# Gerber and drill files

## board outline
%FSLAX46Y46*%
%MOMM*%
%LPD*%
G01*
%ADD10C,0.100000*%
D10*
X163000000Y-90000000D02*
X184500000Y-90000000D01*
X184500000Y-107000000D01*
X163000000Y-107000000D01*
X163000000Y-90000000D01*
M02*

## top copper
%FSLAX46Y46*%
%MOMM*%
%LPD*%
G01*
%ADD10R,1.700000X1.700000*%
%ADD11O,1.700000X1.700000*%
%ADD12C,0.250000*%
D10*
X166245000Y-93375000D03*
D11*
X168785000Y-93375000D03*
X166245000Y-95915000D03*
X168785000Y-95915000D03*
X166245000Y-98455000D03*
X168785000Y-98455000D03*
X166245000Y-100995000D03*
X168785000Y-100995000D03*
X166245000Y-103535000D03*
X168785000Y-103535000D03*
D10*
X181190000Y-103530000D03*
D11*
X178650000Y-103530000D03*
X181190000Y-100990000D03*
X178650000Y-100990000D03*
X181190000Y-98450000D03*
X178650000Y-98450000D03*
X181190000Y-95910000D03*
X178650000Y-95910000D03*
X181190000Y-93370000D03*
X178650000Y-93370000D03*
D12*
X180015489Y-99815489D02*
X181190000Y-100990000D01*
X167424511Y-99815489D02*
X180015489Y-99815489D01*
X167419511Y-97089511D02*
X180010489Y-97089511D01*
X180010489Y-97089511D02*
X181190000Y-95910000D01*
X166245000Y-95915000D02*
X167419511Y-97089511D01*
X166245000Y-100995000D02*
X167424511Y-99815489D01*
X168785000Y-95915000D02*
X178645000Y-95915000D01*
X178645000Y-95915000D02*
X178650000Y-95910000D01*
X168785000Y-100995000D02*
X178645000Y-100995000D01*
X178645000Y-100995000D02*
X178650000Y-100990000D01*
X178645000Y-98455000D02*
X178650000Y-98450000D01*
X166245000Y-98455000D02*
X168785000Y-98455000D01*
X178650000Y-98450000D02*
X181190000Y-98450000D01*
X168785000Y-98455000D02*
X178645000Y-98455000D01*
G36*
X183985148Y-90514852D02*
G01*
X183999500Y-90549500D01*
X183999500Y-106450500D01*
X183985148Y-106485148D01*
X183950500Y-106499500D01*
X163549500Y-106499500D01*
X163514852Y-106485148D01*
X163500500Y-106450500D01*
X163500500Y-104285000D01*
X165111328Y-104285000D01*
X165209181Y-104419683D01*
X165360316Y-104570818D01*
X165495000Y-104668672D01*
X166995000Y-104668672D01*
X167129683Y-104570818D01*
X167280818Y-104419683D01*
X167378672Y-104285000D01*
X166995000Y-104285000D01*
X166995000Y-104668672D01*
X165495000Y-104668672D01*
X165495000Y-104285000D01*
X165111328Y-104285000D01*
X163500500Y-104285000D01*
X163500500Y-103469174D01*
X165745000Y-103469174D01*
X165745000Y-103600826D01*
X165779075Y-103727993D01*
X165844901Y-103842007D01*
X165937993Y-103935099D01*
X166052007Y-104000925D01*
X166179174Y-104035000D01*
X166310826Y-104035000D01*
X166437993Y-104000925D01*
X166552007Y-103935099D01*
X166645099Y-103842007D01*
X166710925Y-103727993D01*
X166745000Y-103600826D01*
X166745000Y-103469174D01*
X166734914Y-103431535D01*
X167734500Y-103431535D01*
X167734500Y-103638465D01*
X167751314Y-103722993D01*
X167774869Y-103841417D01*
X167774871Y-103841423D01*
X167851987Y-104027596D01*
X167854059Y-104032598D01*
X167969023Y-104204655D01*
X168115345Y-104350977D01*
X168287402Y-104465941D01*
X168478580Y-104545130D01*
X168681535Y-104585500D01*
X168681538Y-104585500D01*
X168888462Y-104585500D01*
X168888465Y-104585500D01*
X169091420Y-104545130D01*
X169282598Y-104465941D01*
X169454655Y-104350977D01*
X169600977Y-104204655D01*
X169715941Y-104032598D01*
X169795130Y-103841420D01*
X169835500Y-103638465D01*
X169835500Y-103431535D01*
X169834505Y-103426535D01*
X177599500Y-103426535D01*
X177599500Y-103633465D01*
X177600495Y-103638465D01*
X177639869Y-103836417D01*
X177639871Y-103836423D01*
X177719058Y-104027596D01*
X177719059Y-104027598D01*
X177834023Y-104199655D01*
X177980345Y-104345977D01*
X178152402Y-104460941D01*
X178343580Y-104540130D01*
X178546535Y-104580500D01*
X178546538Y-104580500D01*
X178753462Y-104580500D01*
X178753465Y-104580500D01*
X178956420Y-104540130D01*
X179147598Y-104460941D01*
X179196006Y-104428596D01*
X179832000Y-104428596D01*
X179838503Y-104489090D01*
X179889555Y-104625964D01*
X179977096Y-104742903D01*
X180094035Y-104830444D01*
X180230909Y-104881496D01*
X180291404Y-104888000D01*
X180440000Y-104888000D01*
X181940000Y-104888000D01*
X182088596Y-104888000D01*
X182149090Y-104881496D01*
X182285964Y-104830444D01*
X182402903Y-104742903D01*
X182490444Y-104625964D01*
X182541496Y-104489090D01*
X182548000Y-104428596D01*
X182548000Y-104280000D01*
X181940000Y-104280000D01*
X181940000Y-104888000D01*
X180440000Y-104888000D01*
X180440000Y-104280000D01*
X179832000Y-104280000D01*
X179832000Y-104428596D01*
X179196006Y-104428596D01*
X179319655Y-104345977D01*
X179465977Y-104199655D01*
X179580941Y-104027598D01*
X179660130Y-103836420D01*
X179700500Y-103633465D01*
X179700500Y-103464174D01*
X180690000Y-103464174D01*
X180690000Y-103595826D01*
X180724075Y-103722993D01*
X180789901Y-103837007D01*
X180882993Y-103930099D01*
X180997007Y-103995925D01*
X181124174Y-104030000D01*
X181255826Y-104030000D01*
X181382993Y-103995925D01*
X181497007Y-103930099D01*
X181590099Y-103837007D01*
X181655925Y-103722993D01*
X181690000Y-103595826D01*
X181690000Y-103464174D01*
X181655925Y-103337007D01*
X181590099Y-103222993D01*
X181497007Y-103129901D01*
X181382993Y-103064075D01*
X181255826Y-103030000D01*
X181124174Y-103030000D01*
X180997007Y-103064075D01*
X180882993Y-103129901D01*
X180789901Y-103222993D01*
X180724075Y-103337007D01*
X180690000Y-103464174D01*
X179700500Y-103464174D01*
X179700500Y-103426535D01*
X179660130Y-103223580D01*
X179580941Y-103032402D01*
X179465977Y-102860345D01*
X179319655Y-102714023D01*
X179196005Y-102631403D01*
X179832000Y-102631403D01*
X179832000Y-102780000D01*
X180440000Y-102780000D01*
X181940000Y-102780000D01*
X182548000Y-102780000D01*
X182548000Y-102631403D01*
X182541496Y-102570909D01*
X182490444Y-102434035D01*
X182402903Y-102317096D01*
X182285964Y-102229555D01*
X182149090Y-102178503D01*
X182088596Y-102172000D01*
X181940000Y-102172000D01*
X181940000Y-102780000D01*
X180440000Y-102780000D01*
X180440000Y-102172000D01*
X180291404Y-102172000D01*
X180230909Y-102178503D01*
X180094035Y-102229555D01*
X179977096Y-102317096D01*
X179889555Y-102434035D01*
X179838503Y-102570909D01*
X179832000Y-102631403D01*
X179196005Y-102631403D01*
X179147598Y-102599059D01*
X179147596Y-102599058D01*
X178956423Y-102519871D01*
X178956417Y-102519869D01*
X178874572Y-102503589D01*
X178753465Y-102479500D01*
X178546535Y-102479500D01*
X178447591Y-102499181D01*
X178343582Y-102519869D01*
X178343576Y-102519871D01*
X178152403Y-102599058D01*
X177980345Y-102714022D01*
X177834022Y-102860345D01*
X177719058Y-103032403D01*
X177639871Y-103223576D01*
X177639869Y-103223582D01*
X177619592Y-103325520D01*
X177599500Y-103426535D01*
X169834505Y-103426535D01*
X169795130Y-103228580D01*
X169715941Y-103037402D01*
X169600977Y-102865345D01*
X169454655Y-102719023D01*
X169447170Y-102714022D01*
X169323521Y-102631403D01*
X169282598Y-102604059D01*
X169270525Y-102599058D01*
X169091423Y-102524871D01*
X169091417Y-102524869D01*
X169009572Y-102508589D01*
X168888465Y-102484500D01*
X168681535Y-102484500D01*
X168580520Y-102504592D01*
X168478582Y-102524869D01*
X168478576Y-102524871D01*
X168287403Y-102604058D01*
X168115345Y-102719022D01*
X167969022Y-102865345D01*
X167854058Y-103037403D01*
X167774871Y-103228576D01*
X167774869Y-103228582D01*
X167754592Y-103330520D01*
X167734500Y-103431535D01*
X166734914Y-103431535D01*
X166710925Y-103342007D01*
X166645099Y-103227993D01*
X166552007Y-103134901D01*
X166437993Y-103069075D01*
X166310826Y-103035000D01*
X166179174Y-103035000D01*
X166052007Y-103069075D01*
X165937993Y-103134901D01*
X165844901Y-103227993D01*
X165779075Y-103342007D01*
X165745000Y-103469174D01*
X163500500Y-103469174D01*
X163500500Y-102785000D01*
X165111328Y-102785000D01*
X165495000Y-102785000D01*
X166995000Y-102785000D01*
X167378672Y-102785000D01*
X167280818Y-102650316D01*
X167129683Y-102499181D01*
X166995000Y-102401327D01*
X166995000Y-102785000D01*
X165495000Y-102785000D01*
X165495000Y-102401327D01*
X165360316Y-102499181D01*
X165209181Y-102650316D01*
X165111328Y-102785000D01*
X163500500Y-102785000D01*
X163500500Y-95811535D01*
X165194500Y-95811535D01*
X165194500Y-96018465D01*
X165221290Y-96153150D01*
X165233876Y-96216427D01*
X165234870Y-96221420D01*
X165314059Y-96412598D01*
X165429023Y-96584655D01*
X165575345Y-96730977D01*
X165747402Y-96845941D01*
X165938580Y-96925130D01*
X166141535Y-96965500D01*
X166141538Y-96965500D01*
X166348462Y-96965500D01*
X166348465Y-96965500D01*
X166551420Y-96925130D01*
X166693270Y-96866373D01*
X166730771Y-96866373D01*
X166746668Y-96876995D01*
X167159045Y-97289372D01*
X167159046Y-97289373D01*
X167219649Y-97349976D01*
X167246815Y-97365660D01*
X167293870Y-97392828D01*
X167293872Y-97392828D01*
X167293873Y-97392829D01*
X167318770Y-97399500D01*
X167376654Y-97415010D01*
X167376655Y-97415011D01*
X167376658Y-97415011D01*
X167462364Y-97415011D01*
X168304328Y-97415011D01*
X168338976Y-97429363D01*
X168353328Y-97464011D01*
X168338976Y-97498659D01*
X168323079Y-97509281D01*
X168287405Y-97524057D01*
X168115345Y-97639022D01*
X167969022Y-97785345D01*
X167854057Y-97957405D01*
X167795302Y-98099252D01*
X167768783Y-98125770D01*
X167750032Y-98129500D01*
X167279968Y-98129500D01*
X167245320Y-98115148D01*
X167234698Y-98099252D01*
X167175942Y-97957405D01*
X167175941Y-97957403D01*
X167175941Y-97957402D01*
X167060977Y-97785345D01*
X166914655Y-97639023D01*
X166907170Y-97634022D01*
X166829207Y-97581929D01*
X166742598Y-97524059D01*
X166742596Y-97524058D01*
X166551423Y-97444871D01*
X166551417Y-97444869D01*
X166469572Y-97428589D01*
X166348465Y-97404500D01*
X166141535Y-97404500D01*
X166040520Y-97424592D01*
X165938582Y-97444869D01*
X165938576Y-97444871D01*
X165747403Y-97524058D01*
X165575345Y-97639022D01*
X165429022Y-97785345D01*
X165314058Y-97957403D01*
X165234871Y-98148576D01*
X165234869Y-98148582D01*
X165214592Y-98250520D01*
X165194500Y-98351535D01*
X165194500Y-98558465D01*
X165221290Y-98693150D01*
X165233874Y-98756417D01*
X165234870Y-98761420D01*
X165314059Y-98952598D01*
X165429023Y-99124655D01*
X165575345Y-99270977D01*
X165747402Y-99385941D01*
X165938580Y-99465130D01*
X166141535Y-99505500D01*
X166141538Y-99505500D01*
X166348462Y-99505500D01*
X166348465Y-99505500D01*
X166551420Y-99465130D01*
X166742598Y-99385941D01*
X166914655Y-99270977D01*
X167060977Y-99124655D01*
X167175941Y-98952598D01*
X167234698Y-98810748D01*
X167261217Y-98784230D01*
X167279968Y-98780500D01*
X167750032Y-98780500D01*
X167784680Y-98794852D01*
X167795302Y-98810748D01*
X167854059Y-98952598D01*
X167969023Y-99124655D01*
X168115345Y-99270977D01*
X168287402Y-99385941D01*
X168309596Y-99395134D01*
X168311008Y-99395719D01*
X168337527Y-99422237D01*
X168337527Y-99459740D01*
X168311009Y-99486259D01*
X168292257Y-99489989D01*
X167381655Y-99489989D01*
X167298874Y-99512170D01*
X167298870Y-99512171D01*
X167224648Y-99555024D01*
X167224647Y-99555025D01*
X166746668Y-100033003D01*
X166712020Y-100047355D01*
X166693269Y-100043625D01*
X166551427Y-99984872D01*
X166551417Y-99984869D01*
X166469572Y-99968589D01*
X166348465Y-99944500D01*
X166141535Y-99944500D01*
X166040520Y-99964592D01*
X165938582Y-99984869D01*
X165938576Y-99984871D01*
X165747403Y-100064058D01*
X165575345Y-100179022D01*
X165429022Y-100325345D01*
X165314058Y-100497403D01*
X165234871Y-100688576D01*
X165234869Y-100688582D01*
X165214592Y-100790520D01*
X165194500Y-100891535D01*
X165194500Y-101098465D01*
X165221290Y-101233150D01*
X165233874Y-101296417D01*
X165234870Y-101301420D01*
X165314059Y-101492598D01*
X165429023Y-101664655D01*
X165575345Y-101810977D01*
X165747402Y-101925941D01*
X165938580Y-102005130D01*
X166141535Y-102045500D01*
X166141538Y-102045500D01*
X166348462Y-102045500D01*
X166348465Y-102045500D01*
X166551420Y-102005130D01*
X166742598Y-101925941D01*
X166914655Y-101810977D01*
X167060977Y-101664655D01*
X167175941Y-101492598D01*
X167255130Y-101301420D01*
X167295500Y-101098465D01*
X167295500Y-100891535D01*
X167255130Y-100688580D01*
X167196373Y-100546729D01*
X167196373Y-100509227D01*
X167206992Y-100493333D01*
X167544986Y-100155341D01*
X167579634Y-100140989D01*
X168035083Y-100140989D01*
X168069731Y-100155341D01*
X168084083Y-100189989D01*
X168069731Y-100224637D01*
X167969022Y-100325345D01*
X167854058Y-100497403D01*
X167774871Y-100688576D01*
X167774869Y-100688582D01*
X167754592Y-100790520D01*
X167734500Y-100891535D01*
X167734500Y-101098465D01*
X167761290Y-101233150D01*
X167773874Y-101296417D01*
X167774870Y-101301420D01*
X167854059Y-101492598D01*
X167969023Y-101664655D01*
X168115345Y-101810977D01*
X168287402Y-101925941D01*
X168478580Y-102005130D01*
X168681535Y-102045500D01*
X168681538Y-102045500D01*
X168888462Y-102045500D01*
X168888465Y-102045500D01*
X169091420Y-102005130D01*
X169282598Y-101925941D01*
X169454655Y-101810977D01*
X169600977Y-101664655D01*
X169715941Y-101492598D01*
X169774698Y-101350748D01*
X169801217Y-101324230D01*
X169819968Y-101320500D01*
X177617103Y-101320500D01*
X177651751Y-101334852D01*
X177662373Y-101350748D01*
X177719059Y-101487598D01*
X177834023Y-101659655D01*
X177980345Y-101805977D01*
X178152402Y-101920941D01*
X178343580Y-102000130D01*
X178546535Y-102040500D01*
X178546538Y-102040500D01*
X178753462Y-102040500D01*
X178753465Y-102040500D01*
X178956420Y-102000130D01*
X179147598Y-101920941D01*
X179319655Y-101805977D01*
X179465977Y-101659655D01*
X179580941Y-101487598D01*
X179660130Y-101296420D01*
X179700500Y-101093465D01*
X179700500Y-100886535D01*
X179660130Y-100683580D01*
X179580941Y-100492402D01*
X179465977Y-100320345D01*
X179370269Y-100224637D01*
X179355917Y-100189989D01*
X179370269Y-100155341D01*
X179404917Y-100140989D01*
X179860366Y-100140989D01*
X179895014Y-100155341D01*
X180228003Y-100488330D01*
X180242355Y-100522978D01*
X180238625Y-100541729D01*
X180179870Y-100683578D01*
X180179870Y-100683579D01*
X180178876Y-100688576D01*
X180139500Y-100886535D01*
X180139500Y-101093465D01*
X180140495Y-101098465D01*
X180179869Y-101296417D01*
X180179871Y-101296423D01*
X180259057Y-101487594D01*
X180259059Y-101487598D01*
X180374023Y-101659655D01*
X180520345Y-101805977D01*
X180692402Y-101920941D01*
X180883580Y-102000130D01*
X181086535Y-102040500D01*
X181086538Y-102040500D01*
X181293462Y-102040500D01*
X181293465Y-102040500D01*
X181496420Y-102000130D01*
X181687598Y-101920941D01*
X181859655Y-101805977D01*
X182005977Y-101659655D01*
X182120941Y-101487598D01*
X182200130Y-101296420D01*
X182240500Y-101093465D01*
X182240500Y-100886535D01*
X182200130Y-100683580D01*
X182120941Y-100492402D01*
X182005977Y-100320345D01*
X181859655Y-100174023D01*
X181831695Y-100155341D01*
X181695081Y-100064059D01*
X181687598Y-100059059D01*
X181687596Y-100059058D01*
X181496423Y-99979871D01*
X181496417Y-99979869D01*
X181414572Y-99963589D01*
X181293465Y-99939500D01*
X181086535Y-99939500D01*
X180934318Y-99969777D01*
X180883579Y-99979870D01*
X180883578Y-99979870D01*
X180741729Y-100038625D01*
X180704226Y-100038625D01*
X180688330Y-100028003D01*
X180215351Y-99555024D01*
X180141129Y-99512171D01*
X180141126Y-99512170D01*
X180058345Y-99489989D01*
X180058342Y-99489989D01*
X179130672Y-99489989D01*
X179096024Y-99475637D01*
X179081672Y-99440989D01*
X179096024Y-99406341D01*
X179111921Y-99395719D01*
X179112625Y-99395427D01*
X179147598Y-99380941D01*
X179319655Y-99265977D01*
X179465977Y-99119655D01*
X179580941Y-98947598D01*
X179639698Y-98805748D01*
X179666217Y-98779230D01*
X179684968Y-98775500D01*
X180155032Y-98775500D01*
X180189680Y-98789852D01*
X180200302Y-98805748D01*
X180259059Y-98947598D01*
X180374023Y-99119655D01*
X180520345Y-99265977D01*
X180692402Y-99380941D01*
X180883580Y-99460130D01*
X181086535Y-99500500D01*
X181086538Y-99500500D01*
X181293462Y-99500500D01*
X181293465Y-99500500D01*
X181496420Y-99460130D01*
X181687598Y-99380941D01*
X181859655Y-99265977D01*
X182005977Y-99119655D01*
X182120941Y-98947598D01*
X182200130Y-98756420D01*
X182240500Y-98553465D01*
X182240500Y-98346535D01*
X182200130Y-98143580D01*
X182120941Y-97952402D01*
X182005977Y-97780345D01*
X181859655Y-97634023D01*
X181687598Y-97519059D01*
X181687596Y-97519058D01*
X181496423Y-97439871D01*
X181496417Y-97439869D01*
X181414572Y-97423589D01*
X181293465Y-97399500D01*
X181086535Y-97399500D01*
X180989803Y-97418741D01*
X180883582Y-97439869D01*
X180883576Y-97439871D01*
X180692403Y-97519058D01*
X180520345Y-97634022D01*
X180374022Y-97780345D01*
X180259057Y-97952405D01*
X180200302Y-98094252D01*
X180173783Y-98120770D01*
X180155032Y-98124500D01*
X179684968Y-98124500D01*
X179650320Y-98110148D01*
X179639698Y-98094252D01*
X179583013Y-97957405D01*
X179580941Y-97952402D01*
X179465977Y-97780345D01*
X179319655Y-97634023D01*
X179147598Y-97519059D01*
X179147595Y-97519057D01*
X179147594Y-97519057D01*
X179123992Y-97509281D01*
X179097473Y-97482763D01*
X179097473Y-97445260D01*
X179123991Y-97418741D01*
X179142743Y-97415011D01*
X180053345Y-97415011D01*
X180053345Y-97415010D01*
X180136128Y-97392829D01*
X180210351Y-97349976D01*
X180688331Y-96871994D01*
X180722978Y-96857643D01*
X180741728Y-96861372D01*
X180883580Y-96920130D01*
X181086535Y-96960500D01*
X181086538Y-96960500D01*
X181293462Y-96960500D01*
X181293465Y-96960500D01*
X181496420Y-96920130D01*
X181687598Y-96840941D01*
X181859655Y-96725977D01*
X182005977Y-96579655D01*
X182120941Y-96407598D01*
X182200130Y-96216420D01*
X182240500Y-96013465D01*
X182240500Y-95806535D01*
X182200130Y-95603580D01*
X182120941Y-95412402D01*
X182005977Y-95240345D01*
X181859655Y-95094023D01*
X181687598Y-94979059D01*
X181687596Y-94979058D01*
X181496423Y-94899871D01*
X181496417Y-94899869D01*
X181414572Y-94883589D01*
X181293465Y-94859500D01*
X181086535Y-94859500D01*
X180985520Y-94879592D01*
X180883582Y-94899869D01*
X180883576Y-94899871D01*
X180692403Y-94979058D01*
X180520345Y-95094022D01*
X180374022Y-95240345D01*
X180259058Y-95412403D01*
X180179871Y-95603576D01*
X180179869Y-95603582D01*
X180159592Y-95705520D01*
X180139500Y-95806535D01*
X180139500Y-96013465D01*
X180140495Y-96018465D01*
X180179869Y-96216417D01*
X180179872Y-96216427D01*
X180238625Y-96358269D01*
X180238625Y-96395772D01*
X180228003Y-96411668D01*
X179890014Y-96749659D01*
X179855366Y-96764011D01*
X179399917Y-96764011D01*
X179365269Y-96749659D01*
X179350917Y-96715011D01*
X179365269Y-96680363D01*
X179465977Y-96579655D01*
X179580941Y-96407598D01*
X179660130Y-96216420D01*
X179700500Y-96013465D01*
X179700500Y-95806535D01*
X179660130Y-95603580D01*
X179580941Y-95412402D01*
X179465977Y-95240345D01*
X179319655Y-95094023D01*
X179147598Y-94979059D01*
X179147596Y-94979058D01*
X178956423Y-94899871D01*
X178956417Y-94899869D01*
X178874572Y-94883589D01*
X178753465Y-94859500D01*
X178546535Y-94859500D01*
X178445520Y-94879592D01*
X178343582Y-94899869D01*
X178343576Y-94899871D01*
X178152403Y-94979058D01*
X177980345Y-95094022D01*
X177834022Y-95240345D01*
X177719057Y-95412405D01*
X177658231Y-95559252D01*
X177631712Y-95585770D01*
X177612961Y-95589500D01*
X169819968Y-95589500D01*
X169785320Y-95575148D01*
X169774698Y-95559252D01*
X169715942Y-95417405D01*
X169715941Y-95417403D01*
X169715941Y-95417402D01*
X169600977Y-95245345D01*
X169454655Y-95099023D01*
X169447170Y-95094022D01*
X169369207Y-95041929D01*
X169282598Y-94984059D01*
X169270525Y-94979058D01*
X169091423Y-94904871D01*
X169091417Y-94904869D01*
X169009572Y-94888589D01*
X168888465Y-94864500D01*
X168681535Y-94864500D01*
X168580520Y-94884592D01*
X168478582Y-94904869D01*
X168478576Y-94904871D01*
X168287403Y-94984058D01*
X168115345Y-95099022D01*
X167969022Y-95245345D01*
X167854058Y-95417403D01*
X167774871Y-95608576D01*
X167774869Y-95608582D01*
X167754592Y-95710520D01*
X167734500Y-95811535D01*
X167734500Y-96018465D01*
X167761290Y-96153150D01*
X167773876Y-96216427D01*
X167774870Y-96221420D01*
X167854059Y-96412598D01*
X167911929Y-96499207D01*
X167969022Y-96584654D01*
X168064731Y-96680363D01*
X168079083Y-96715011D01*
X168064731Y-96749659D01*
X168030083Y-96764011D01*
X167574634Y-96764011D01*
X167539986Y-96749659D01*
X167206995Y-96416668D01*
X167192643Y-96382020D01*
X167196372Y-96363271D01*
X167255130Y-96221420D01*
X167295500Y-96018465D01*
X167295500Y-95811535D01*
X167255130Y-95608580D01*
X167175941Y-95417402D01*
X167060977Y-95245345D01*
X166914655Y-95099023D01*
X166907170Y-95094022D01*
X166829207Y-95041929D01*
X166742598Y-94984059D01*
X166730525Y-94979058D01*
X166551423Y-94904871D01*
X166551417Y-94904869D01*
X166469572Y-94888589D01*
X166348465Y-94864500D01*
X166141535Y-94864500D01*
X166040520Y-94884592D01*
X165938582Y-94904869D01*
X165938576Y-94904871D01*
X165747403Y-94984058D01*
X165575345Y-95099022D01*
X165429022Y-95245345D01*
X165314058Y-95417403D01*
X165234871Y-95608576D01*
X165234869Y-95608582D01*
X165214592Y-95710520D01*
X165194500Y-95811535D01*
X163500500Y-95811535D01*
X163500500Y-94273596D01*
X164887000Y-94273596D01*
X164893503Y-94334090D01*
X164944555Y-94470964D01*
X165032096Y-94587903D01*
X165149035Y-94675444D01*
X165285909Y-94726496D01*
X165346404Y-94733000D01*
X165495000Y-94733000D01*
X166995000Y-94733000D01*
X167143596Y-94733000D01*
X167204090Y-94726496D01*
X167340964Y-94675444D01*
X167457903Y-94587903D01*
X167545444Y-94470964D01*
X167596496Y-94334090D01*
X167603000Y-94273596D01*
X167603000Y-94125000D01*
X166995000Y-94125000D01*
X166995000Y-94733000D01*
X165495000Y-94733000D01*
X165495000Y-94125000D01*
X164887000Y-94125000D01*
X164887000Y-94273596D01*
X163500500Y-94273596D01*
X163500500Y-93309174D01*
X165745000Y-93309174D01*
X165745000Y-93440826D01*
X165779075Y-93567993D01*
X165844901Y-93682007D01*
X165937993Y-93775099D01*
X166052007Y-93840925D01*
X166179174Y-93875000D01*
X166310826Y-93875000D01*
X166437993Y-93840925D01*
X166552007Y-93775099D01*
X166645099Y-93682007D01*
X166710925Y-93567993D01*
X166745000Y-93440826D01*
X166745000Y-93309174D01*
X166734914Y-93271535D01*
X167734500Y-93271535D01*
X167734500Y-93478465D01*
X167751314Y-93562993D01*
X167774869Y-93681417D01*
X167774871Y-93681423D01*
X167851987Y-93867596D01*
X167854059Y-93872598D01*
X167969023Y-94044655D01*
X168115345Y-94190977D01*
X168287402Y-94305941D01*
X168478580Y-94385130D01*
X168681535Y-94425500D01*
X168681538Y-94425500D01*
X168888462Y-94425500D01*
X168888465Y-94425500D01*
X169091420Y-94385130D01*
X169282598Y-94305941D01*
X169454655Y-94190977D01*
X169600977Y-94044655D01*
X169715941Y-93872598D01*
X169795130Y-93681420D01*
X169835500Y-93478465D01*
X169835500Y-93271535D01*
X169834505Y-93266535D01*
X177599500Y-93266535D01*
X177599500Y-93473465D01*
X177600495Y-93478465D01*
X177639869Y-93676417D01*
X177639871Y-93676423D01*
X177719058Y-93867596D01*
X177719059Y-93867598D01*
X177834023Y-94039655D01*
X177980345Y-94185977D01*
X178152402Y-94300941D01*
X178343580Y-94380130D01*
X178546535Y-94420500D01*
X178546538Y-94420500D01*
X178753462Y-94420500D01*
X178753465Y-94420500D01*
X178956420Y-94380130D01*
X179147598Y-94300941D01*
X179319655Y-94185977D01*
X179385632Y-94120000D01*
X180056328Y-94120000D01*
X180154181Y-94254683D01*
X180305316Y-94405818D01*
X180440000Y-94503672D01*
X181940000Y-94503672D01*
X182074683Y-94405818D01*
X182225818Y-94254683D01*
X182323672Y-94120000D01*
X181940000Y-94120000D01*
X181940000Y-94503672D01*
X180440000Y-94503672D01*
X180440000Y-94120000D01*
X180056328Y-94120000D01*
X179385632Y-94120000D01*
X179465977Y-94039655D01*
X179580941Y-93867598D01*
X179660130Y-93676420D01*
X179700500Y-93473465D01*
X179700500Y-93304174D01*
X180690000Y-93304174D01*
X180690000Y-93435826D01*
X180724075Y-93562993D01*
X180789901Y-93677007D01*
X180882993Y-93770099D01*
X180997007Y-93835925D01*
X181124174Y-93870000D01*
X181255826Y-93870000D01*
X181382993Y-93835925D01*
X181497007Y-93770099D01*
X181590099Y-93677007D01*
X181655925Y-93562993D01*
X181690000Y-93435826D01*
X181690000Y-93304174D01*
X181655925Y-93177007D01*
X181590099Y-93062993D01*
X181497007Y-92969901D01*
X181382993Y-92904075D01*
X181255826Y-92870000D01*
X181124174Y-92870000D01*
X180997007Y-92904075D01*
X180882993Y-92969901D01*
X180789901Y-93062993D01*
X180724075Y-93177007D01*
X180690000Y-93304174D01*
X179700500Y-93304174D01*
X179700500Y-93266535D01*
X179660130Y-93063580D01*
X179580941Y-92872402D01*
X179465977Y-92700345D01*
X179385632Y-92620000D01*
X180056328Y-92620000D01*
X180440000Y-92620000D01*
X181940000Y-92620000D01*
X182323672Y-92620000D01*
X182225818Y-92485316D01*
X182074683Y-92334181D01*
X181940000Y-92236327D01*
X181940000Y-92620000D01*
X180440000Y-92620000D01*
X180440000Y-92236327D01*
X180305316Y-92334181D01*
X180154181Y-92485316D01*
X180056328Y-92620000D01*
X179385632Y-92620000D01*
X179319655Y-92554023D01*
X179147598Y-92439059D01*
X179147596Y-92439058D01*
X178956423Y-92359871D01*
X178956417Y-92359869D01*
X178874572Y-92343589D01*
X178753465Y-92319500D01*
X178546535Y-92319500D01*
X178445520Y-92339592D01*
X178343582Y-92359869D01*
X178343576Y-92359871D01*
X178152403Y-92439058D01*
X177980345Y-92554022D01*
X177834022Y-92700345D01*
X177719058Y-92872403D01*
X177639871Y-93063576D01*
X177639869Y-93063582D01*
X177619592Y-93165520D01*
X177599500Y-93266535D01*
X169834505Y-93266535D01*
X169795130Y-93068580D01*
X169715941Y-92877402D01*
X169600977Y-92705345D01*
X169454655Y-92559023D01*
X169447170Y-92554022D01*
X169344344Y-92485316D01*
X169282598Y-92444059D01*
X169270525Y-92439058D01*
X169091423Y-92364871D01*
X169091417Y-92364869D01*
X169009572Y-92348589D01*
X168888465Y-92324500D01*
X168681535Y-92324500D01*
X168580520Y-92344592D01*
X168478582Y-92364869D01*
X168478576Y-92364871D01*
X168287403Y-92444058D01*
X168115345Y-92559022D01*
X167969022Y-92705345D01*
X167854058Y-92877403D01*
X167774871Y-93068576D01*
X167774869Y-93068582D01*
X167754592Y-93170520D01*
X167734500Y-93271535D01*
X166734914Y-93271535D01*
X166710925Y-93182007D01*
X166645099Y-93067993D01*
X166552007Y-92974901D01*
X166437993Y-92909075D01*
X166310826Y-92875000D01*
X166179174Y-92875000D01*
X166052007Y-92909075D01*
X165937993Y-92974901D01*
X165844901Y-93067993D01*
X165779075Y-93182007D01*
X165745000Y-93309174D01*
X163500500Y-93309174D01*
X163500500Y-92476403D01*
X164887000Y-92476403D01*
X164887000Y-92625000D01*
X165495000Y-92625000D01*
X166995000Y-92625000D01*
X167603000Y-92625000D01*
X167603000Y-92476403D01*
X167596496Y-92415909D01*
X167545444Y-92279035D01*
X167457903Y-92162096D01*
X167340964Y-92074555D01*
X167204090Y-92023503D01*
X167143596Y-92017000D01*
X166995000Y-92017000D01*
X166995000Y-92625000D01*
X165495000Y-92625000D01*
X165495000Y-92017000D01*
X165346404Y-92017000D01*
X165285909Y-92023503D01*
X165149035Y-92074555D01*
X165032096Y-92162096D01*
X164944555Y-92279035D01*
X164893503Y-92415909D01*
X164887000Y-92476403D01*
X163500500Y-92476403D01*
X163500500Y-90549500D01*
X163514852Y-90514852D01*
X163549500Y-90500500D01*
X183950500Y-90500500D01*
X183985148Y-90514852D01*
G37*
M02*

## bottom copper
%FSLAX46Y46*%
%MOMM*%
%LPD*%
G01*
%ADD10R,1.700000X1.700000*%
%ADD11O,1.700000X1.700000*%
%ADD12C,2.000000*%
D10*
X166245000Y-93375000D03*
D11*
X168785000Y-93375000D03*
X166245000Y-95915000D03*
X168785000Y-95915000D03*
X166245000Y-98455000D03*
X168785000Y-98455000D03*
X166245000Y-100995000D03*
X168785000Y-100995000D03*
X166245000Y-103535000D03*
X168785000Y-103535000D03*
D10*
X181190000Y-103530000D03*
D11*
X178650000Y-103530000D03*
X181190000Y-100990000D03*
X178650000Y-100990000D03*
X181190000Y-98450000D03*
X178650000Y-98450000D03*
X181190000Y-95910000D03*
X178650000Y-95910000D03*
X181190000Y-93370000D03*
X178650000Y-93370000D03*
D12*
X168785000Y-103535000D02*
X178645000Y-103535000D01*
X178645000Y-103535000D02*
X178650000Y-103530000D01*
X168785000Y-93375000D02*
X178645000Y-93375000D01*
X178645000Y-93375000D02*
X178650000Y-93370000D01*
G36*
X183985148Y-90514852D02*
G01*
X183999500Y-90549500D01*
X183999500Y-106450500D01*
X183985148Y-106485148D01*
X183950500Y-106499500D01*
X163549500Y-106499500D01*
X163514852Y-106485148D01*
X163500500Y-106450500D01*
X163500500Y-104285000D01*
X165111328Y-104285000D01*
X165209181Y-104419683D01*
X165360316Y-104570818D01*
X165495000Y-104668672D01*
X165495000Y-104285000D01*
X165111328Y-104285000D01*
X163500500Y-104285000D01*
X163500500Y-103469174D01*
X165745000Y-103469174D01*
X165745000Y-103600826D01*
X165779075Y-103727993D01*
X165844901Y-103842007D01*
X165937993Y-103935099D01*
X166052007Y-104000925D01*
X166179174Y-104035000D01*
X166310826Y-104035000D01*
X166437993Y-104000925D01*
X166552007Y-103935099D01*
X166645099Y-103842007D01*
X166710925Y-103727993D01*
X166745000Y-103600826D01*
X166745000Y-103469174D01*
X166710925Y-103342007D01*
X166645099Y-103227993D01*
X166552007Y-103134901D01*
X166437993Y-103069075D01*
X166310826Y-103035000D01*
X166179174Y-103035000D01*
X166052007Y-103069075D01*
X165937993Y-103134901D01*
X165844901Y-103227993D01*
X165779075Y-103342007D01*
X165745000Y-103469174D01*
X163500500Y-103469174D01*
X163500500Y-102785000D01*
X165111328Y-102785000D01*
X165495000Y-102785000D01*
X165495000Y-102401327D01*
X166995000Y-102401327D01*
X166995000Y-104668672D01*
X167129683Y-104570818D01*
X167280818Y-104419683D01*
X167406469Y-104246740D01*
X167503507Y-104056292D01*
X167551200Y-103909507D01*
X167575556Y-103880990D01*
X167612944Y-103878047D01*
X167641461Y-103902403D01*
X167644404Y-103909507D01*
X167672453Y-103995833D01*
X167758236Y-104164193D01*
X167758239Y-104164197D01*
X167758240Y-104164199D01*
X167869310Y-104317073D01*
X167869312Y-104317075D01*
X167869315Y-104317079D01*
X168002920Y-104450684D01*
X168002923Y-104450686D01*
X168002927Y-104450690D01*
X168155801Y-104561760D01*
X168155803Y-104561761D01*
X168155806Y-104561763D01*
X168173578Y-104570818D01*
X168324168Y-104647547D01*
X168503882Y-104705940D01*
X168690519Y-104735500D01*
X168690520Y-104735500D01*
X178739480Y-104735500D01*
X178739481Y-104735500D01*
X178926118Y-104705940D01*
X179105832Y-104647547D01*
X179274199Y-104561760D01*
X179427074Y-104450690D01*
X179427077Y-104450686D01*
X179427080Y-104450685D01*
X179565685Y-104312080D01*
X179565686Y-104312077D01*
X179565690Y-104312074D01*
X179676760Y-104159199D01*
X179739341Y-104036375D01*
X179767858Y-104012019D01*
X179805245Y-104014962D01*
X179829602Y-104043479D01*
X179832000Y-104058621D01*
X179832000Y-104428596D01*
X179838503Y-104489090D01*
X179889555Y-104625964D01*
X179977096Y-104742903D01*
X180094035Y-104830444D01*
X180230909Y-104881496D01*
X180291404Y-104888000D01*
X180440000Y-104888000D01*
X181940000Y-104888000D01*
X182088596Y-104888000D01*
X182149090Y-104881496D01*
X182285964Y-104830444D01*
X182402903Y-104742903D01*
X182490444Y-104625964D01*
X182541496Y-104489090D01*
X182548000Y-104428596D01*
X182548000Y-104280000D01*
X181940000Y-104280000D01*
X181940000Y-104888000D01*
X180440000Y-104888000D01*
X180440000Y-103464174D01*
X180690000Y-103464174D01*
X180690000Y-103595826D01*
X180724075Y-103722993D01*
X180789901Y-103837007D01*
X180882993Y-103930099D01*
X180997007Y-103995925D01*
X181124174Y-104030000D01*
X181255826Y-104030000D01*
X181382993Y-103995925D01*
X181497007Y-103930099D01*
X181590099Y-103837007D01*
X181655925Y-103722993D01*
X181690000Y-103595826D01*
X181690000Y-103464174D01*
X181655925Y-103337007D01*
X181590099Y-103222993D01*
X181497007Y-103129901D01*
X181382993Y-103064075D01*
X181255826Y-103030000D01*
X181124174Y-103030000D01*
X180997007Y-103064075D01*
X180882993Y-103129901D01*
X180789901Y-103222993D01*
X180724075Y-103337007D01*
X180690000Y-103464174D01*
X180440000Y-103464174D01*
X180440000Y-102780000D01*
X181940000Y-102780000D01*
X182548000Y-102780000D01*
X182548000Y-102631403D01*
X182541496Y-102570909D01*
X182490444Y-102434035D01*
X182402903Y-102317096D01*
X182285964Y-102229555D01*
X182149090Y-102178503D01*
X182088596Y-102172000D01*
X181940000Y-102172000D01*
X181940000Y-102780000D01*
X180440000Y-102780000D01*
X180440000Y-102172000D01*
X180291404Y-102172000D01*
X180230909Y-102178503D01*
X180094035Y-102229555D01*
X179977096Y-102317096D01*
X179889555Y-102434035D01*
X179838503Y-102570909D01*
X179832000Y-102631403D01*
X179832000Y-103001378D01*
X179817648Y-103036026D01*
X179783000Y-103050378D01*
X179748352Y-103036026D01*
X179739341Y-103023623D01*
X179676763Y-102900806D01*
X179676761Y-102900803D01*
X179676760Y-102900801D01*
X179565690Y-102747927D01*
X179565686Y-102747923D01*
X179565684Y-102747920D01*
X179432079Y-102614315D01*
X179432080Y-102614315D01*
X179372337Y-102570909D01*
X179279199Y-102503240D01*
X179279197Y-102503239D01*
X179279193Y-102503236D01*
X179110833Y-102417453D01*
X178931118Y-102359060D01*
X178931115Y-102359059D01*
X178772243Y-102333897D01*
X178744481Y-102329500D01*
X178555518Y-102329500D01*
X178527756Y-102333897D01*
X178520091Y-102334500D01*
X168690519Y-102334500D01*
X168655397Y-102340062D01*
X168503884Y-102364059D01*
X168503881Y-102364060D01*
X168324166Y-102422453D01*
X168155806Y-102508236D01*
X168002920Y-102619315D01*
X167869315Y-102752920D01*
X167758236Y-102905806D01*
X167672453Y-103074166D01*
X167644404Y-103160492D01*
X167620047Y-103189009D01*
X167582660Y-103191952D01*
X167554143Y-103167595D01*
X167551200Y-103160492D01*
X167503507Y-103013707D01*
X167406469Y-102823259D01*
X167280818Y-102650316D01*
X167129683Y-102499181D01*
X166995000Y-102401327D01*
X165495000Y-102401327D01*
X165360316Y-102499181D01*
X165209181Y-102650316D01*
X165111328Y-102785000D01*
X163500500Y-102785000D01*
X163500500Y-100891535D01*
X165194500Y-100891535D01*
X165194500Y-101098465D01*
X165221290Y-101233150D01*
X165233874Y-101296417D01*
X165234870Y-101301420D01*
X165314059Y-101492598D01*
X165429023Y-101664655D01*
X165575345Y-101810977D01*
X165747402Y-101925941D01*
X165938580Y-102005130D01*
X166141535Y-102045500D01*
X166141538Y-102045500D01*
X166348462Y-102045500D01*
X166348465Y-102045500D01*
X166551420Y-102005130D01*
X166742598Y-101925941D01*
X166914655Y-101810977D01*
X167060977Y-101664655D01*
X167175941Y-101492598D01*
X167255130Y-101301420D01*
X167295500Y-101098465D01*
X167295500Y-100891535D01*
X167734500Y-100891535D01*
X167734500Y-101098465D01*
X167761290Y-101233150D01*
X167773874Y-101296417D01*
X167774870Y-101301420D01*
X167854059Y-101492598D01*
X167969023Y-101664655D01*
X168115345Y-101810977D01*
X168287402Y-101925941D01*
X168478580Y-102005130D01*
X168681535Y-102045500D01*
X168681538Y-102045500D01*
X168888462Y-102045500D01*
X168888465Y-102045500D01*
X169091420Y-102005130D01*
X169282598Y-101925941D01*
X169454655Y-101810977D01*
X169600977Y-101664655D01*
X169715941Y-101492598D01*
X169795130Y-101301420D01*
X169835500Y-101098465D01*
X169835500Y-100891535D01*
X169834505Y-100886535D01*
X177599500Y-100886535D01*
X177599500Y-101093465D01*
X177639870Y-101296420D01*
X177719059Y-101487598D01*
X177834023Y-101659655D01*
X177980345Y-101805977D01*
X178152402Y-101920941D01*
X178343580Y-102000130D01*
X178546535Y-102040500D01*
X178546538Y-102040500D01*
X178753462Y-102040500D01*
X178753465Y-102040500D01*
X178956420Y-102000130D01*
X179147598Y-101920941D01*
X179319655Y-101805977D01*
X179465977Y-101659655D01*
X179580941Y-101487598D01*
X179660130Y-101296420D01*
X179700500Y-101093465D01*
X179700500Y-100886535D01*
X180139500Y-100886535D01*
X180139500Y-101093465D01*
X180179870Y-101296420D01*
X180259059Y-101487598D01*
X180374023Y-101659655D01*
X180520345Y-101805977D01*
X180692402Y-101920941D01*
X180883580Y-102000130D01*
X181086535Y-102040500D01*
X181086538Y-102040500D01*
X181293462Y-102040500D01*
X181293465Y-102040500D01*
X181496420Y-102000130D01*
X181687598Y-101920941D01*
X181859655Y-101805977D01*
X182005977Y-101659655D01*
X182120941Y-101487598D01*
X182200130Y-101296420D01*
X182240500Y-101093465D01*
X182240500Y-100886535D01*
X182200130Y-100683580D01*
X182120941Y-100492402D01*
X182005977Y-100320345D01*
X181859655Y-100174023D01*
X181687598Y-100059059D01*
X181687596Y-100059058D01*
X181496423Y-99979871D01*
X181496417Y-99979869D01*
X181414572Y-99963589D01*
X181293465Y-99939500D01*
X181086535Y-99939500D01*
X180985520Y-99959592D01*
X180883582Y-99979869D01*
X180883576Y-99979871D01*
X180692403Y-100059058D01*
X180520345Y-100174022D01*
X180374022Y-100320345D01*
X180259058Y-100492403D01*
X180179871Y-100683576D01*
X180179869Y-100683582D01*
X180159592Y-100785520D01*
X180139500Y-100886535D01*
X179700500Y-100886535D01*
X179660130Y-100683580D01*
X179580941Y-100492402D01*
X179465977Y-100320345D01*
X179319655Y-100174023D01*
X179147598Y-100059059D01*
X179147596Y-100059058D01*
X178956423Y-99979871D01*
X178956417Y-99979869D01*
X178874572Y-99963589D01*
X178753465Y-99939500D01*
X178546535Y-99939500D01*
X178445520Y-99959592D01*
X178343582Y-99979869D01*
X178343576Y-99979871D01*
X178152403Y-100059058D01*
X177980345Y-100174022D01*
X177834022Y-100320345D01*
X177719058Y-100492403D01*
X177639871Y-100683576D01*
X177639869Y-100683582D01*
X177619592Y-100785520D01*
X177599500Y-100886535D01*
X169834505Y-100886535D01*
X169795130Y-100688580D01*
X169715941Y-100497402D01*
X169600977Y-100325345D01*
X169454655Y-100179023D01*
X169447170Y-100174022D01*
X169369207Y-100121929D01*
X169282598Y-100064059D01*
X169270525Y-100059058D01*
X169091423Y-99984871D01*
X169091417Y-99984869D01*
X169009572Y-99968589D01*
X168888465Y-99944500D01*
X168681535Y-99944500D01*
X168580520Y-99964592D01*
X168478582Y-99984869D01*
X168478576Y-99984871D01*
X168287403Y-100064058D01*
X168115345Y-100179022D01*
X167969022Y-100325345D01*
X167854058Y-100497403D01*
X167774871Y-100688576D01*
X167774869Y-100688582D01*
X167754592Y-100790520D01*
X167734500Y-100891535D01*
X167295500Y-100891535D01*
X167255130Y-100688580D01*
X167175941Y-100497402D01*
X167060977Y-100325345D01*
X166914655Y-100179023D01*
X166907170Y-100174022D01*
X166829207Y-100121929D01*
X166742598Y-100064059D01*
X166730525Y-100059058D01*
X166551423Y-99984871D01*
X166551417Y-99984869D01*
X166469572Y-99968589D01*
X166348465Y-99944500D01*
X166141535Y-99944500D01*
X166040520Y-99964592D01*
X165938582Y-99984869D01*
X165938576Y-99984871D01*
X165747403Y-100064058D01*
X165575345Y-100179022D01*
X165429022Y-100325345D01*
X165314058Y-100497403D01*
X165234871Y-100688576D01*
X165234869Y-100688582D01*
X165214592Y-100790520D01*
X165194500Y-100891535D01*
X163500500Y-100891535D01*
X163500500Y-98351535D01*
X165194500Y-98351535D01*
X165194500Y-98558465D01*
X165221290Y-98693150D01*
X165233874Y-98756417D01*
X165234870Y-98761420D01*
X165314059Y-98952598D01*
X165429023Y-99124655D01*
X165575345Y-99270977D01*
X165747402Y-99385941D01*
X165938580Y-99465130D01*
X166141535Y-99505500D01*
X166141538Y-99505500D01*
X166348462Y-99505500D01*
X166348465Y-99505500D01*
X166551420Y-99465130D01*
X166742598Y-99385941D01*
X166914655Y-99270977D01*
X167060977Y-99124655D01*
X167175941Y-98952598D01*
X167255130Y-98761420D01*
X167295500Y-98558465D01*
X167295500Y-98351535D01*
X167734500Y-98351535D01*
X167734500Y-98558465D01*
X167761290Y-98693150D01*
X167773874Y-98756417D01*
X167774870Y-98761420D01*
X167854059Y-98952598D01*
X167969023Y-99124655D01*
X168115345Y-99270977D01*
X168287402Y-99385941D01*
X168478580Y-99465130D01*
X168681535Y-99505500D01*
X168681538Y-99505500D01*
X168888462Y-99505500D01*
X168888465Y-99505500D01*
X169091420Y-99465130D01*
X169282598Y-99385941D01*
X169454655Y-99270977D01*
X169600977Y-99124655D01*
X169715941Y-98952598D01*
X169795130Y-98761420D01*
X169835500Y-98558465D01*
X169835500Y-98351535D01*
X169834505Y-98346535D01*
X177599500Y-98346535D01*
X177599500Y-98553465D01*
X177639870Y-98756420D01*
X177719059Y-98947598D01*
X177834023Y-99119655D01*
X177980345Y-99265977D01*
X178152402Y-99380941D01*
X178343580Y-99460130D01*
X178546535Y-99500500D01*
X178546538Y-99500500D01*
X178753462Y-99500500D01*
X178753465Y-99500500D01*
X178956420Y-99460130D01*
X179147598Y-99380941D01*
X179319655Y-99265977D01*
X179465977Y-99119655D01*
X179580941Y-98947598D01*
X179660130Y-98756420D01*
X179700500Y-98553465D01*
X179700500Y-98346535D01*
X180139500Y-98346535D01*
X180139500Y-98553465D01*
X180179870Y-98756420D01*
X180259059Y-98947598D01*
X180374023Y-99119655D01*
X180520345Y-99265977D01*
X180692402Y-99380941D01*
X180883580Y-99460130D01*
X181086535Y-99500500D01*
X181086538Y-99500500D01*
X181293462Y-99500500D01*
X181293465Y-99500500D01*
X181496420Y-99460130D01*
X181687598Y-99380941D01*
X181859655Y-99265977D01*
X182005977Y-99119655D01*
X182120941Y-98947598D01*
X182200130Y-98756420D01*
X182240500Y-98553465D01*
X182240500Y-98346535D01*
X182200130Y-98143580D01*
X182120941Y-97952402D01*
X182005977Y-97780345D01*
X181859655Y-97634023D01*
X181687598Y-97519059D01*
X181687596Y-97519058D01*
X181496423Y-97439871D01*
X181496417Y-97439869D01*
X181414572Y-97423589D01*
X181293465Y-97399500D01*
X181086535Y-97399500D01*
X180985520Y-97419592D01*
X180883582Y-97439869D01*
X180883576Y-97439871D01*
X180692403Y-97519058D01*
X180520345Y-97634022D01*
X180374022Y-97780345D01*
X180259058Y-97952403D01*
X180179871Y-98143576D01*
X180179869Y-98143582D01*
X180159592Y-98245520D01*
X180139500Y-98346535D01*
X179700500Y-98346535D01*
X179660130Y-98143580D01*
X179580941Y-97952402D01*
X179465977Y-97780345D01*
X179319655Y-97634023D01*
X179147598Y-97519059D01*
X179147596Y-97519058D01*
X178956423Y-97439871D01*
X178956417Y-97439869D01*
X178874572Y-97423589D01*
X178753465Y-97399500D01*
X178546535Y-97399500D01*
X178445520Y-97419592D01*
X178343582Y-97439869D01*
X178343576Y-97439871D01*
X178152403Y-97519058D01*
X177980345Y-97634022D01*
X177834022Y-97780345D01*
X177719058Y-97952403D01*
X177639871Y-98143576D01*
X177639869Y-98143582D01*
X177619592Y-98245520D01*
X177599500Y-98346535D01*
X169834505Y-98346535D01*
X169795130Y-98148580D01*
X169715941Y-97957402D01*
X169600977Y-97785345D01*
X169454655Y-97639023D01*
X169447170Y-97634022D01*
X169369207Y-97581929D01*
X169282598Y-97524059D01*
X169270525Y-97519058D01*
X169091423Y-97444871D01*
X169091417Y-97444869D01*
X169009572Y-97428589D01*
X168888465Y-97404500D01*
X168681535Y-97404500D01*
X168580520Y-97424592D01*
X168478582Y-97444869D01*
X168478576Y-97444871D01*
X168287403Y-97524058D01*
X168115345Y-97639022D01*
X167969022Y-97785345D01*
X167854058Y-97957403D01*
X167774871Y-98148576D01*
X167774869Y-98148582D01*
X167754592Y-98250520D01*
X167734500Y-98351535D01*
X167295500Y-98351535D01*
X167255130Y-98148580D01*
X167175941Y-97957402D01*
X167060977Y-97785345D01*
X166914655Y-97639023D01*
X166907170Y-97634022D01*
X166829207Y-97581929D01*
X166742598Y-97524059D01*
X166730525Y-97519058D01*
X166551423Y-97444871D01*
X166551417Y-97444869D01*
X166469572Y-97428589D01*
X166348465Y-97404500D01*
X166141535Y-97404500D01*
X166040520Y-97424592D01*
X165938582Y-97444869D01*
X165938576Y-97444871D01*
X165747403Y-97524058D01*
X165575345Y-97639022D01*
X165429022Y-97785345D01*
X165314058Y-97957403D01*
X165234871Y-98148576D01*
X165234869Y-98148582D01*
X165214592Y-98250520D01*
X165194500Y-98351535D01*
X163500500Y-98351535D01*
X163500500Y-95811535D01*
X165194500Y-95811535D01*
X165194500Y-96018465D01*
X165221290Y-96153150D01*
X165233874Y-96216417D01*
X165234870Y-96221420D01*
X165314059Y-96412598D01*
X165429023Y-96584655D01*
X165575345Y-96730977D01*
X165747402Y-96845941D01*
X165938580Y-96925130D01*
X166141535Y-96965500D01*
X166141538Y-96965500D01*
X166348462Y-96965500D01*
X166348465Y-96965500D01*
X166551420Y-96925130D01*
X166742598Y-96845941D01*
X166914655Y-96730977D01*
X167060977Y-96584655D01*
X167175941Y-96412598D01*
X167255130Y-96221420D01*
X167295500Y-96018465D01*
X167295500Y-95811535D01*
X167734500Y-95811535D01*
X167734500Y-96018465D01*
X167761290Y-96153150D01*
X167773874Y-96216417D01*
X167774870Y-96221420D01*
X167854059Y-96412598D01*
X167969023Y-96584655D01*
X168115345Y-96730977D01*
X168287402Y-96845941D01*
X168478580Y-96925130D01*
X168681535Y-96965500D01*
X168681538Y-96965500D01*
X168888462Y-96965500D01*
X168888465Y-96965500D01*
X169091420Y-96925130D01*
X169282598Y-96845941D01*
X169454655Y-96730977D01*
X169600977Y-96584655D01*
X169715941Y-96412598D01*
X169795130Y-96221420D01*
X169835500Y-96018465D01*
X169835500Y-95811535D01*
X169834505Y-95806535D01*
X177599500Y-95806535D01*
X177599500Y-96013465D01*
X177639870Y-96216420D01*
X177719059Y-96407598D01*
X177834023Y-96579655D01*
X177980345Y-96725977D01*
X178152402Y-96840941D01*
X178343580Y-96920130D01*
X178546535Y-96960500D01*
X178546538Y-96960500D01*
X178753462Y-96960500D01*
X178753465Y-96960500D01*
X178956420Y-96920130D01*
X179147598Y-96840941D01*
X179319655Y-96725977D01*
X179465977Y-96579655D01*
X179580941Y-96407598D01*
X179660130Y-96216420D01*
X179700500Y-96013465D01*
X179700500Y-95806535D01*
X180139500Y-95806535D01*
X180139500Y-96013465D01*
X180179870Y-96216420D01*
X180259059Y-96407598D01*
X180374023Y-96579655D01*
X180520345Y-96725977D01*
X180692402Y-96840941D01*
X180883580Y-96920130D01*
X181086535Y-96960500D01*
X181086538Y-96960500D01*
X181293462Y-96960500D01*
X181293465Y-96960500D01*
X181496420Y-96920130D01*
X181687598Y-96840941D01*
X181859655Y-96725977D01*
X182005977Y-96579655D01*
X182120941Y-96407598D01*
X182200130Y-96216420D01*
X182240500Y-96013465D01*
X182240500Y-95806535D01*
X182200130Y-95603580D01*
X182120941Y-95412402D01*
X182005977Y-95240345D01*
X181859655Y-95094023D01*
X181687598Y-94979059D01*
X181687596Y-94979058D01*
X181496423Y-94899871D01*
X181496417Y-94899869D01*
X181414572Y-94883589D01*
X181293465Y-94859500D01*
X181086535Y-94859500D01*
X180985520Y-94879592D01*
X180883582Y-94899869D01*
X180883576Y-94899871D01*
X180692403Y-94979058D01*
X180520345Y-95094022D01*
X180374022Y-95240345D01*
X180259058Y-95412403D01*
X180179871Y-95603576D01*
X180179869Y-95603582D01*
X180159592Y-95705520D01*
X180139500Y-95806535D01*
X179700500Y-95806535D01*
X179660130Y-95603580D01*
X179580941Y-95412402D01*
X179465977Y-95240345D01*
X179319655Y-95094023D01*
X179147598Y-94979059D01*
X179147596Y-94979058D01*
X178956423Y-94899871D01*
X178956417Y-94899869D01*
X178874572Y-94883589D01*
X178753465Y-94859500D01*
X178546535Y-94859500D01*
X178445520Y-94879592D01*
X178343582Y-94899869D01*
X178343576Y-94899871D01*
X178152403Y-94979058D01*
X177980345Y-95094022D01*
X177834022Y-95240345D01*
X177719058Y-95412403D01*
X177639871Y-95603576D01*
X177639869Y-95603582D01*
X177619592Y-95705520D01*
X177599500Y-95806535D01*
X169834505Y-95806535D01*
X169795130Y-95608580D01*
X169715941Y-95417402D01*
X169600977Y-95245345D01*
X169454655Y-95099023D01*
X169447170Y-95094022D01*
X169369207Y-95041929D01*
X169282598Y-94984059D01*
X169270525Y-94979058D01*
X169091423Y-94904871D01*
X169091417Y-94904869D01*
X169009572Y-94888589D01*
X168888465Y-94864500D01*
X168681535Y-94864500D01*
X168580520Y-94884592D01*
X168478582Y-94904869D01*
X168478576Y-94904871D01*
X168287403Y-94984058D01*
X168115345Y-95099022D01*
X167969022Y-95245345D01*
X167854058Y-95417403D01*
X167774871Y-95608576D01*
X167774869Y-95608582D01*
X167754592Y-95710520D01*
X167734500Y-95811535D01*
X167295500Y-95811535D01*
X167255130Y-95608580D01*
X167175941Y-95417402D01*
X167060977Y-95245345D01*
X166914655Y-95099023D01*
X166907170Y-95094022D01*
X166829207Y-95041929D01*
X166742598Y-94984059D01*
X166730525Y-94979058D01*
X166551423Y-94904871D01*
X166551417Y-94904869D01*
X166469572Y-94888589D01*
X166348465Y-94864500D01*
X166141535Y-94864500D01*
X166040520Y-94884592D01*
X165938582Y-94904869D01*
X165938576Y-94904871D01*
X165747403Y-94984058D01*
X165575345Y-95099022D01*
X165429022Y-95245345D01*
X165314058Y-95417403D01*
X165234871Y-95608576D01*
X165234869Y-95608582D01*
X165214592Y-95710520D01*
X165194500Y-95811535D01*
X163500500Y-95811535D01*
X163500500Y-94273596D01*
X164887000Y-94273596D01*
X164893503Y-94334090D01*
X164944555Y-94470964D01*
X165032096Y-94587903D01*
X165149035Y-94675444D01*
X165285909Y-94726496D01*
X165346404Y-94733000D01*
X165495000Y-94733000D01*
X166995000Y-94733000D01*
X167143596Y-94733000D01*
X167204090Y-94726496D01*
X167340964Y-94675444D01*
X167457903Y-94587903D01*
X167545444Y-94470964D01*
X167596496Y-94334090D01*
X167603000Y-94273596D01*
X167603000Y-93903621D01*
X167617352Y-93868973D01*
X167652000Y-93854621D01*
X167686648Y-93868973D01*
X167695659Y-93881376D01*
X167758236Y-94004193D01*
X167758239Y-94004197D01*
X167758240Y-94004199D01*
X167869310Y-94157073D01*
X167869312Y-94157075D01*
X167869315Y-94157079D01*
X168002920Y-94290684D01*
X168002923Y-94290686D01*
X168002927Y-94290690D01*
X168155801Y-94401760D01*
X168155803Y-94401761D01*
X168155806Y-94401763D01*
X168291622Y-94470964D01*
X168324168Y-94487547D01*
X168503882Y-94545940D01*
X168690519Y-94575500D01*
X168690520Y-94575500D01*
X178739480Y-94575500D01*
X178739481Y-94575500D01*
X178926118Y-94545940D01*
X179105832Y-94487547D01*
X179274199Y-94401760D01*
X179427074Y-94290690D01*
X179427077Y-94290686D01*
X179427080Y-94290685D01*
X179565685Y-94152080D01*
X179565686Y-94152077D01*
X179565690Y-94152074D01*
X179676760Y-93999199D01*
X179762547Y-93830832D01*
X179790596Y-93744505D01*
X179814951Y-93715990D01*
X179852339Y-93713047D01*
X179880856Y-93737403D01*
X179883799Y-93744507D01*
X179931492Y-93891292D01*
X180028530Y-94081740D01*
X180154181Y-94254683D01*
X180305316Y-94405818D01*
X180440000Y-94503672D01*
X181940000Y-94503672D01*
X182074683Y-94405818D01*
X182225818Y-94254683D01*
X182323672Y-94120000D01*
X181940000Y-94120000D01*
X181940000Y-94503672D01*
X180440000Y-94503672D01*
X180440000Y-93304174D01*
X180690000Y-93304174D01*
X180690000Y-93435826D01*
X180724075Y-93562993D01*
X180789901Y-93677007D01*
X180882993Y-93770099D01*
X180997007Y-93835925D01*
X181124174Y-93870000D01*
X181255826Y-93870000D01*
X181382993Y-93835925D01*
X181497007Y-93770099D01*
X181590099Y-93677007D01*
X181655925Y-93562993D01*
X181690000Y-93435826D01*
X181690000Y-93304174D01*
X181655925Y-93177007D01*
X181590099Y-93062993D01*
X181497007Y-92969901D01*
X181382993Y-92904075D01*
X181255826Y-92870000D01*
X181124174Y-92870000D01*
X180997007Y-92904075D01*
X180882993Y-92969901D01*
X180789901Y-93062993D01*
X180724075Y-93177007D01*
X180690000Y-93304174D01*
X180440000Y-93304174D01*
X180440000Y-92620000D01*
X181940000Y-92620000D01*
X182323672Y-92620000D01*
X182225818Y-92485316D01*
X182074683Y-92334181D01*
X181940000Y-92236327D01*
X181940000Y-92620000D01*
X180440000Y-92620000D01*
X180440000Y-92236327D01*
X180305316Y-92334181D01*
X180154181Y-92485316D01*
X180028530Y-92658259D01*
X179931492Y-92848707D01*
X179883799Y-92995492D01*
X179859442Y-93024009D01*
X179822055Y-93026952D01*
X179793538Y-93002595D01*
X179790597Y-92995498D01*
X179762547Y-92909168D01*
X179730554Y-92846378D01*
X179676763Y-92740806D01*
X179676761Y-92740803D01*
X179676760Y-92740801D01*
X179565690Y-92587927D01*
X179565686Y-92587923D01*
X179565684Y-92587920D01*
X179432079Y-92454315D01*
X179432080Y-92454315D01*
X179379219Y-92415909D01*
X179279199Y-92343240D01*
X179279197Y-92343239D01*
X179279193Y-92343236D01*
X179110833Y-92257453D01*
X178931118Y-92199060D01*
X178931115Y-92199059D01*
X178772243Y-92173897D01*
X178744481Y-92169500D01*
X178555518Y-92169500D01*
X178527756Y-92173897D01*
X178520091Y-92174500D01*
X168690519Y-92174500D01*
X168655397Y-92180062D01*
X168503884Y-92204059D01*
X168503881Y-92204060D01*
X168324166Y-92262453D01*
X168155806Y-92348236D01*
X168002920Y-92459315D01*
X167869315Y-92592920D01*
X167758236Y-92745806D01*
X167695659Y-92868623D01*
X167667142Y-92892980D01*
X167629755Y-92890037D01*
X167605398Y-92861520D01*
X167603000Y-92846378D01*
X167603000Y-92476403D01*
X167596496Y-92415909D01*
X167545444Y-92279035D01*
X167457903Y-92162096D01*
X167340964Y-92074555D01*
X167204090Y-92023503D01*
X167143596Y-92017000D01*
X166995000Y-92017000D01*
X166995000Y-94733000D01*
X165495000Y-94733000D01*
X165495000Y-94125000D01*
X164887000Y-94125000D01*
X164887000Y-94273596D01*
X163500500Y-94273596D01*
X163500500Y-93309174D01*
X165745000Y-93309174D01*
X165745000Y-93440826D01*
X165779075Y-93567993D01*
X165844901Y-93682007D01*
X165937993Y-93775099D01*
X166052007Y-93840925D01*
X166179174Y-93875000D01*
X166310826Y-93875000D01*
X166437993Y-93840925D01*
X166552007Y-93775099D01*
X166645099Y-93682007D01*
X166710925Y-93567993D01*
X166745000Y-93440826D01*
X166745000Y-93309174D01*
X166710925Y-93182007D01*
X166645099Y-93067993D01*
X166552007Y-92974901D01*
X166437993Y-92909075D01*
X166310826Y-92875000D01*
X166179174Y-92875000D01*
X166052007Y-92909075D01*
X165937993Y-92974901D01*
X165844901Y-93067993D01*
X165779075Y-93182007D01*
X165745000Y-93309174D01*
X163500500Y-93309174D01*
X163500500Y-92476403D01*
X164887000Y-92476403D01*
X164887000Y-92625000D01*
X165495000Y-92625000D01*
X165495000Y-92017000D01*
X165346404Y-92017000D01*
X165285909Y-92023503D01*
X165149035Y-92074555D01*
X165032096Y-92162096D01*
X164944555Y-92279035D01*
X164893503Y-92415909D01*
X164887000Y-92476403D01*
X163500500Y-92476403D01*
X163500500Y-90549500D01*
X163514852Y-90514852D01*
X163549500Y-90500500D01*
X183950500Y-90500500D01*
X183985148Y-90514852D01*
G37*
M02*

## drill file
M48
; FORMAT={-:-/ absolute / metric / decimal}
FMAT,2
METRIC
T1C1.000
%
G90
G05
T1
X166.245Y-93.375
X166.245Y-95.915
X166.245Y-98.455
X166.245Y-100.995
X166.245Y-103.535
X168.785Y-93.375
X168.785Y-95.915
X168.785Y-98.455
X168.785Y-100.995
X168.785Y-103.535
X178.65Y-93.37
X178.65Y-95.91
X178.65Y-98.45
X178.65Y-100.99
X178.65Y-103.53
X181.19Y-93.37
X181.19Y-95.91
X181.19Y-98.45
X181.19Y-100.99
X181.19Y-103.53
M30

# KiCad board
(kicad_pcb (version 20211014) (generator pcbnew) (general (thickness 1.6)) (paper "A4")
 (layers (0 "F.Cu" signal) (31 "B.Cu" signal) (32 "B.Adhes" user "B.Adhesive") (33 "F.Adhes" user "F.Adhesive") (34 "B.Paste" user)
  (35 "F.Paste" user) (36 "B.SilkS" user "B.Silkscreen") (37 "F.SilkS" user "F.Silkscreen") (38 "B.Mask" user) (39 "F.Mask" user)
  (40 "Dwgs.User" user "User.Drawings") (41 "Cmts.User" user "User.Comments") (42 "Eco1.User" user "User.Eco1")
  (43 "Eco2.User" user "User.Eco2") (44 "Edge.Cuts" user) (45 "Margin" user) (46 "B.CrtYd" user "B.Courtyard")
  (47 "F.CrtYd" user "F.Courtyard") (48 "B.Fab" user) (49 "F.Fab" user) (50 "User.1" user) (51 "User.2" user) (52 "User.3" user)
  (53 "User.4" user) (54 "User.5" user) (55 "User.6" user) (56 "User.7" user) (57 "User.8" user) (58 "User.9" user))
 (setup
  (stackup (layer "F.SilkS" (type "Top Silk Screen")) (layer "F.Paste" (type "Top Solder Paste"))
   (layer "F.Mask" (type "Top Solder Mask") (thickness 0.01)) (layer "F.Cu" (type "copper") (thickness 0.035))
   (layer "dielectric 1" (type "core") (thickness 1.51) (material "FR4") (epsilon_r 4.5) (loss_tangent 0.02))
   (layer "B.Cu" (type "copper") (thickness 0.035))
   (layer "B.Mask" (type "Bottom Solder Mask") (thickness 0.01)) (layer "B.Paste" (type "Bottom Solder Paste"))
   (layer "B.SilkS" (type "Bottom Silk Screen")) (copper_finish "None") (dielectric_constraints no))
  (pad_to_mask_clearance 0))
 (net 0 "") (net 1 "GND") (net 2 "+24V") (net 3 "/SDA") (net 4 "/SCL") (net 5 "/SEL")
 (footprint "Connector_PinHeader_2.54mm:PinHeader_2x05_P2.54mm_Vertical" (layer "F.Cu") (at 166.245 93.375)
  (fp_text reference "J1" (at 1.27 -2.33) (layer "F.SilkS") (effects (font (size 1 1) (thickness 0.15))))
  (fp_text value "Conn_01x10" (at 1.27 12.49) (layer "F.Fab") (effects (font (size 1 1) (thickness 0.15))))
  (pad "1" thru_hole rect (at 0 0) (size 1.7 1.7) (drill 1) (layers *.Cu *.Mask) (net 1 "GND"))
  (pad "2" thru_hole oval (at 2.54 0) (size 1.7 1.7) (drill 1) (layers *.Cu *.Mask) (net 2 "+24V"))
  (pad "3" thru_hole oval (at 0 2.54) (size 1.7 1.7) (drill 1) (layers *.Cu *.Mask) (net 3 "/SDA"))
  (pad "4" thru_hole oval (at 2.54 2.54) (size 1.7 1.7) (drill 1) (layers *.Cu *.Mask) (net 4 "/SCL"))
  (pad "5" thru_hole oval (at 0 5.08) (size 1.7 1.7) (drill 1) (layers *.Cu *.Mask) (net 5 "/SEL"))
  (pad "6" thru_hole oval (at 2.54 5.08) (size 1.7 1.7) (drill 1) (layers *.Cu *.Mask) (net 5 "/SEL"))
  (pad "7" thru_hole oval (at 0 7.62) (size 1.7 1.7) (drill 1) (layers *.Cu *.Mask) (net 3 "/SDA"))
  (pad "8" thru_hole oval (at 2.54 7.62) (size 1.7 1.7) (drill 1) (layers *.Cu *.Mask) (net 4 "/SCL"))
  (pad "9" thru_hole oval (at 0 10.16) (size 1.7 1.7) (drill 1) (layers *.Cu *.Mask) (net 1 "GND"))
  (pad "10" thru_hole oval (at 2.54 10.16) (size 1.7 1.7) (drill 1) (layers *.Cu *.Mask) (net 2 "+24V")))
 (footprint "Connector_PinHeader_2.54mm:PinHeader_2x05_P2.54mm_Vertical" (layer "F.Cu") (at 181.19 103.53 180)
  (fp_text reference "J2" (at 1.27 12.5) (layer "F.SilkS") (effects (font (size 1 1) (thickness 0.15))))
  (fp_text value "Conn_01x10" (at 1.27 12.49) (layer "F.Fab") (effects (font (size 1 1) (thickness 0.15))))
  (pad "1" thru_hole rect (at 0 0 180) (size 1.7 1.7) (drill 1) (layers *.Cu *.Mask) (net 1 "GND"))
  (pad "2" thru_hole oval (at 2.54 0 180) (size 1.7 1.7) (drill 1) (layers *.Cu *.Mask) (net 2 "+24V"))
  (pad "3" thru_hole oval (at 0 2.54 180) (size 1.7 1.7) (drill 1) (layers *.Cu *.Mask) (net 3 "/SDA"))
  (pad "4" thru_hole oval (at 2.54 2.54 180) (size 1.7 1.7) (drill 1) (layers *.Cu *.Mask) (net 4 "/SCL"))
  (pad "5" thru_hole oval (at 0 5.08 180) (size 1.7 1.7) (drill 1) (layers *.Cu *.Mask) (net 5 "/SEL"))
  (pad "6" thru_hole oval (at 2.54 5.08 180) (size 1.7 1.7) (drill 1) (layers *.Cu *.Mask) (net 5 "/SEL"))
  (pad "7" thru_hole oval (at 0 7.62 180) (size 1.7 1.7) (drill 1) (layers *.Cu *.Mask) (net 3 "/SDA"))
  (pad "8" thru_hole oval (at 2.54 7.62 180) (size 1.7 1.7) (drill 1) (layers *.Cu *.Mask) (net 4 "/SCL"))
  (pad "9" thru_hole oval (at 0 10.16 180) (size 1.7 1.7) (drill 1) (layers *.Cu *.Mask) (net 1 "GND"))
  (pad "10" thru_hole oval (at 2.54 10.16 180) (size 1.7 1.7) (drill 1) (layers *.Cu *.Mask) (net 2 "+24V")))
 (gr_rect (start 163 90) (end 184.5 107) (layer "Edge.Cuts") (width 0.1) (fill none))
 (segment (start 168.785 103.535) (end 178.645 103.535) (width 2) (layer "B.Cu") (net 2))
 (segment (start 178.645 103.535) (end 178.65 103.53) (width 2) (layer "B.Cu") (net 2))
 (segment (start 168.785 93.375) (end 178.645 93.375) (width 2) (layer "B.Cu") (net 2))
 (segment (start 178.645 93.375) (end 178.65 93.37) (width 2) (layer "B.Cu") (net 2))
 (segment (start 180.015489 99.815489) (end 181.19 100.99) (width 0.25) (layer "F.Cu") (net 3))
 (segment (start 167.424511 99.815489) (end 180.015489 99.815489) (width 0.25) (layer "F.Cu") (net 3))
 (segment (start 167.419511 97.089511) (end 180.010489 97.089511) (width 0.25) (layer "F.Cu") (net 3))
 (segment (start 180.010489 97.089511) (end 181.19 95.91) (width 0.25) (layer "F.Cu") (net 3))
 (segment (start 166.245 95.915) (end 167.419511 97.089511) (width 0.25) (layer "F.Cu") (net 3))
 (segment (start 166.245 100.995) (end 167.424511 99.815489) (width 0.25) (layer "F.Cu") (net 3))
 (segment (start 168.785 95.915) (end 178.645 95.915) (width 0.25) (layer "F.Cu") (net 4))
 (segment (start 178.645 95.915) (end 178.65 95.91) (width 0.25) (layer "F.Cu") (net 4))
 (segment (start 168.785 100.995) (end 178.645 100.995) (width 0.25) (layer "F.Cu") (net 4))
 (segment (start 178.645 100.995) (end 178.65 100.99) (width 0.25) (layer "F.Cu") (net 4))
 (segment (start 178.645 98.455) (end 178.65 98.45) (width 0.25) (layer "F.Cu") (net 5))
 (segment (start 166.245 98.455) (end 168.785 98.455) (width 0.25) (layer "F.Cu") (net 5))
 (segment (start 178.65 98.45) (end 181.19 98.45) (width 0.25) (layer "F.Cu") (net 5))
 (segment (start 168.785 98.455) (end 178.645 98.455) (width 0.25) (layer "F.Cu") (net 5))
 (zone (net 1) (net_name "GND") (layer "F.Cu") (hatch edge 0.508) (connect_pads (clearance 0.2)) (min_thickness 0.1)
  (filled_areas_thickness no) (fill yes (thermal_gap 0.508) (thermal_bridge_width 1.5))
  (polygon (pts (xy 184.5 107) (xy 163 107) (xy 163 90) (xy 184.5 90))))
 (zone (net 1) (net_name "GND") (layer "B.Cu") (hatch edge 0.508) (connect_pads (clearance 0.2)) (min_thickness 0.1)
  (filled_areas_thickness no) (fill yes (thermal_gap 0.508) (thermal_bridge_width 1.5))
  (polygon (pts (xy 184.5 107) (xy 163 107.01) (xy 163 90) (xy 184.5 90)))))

